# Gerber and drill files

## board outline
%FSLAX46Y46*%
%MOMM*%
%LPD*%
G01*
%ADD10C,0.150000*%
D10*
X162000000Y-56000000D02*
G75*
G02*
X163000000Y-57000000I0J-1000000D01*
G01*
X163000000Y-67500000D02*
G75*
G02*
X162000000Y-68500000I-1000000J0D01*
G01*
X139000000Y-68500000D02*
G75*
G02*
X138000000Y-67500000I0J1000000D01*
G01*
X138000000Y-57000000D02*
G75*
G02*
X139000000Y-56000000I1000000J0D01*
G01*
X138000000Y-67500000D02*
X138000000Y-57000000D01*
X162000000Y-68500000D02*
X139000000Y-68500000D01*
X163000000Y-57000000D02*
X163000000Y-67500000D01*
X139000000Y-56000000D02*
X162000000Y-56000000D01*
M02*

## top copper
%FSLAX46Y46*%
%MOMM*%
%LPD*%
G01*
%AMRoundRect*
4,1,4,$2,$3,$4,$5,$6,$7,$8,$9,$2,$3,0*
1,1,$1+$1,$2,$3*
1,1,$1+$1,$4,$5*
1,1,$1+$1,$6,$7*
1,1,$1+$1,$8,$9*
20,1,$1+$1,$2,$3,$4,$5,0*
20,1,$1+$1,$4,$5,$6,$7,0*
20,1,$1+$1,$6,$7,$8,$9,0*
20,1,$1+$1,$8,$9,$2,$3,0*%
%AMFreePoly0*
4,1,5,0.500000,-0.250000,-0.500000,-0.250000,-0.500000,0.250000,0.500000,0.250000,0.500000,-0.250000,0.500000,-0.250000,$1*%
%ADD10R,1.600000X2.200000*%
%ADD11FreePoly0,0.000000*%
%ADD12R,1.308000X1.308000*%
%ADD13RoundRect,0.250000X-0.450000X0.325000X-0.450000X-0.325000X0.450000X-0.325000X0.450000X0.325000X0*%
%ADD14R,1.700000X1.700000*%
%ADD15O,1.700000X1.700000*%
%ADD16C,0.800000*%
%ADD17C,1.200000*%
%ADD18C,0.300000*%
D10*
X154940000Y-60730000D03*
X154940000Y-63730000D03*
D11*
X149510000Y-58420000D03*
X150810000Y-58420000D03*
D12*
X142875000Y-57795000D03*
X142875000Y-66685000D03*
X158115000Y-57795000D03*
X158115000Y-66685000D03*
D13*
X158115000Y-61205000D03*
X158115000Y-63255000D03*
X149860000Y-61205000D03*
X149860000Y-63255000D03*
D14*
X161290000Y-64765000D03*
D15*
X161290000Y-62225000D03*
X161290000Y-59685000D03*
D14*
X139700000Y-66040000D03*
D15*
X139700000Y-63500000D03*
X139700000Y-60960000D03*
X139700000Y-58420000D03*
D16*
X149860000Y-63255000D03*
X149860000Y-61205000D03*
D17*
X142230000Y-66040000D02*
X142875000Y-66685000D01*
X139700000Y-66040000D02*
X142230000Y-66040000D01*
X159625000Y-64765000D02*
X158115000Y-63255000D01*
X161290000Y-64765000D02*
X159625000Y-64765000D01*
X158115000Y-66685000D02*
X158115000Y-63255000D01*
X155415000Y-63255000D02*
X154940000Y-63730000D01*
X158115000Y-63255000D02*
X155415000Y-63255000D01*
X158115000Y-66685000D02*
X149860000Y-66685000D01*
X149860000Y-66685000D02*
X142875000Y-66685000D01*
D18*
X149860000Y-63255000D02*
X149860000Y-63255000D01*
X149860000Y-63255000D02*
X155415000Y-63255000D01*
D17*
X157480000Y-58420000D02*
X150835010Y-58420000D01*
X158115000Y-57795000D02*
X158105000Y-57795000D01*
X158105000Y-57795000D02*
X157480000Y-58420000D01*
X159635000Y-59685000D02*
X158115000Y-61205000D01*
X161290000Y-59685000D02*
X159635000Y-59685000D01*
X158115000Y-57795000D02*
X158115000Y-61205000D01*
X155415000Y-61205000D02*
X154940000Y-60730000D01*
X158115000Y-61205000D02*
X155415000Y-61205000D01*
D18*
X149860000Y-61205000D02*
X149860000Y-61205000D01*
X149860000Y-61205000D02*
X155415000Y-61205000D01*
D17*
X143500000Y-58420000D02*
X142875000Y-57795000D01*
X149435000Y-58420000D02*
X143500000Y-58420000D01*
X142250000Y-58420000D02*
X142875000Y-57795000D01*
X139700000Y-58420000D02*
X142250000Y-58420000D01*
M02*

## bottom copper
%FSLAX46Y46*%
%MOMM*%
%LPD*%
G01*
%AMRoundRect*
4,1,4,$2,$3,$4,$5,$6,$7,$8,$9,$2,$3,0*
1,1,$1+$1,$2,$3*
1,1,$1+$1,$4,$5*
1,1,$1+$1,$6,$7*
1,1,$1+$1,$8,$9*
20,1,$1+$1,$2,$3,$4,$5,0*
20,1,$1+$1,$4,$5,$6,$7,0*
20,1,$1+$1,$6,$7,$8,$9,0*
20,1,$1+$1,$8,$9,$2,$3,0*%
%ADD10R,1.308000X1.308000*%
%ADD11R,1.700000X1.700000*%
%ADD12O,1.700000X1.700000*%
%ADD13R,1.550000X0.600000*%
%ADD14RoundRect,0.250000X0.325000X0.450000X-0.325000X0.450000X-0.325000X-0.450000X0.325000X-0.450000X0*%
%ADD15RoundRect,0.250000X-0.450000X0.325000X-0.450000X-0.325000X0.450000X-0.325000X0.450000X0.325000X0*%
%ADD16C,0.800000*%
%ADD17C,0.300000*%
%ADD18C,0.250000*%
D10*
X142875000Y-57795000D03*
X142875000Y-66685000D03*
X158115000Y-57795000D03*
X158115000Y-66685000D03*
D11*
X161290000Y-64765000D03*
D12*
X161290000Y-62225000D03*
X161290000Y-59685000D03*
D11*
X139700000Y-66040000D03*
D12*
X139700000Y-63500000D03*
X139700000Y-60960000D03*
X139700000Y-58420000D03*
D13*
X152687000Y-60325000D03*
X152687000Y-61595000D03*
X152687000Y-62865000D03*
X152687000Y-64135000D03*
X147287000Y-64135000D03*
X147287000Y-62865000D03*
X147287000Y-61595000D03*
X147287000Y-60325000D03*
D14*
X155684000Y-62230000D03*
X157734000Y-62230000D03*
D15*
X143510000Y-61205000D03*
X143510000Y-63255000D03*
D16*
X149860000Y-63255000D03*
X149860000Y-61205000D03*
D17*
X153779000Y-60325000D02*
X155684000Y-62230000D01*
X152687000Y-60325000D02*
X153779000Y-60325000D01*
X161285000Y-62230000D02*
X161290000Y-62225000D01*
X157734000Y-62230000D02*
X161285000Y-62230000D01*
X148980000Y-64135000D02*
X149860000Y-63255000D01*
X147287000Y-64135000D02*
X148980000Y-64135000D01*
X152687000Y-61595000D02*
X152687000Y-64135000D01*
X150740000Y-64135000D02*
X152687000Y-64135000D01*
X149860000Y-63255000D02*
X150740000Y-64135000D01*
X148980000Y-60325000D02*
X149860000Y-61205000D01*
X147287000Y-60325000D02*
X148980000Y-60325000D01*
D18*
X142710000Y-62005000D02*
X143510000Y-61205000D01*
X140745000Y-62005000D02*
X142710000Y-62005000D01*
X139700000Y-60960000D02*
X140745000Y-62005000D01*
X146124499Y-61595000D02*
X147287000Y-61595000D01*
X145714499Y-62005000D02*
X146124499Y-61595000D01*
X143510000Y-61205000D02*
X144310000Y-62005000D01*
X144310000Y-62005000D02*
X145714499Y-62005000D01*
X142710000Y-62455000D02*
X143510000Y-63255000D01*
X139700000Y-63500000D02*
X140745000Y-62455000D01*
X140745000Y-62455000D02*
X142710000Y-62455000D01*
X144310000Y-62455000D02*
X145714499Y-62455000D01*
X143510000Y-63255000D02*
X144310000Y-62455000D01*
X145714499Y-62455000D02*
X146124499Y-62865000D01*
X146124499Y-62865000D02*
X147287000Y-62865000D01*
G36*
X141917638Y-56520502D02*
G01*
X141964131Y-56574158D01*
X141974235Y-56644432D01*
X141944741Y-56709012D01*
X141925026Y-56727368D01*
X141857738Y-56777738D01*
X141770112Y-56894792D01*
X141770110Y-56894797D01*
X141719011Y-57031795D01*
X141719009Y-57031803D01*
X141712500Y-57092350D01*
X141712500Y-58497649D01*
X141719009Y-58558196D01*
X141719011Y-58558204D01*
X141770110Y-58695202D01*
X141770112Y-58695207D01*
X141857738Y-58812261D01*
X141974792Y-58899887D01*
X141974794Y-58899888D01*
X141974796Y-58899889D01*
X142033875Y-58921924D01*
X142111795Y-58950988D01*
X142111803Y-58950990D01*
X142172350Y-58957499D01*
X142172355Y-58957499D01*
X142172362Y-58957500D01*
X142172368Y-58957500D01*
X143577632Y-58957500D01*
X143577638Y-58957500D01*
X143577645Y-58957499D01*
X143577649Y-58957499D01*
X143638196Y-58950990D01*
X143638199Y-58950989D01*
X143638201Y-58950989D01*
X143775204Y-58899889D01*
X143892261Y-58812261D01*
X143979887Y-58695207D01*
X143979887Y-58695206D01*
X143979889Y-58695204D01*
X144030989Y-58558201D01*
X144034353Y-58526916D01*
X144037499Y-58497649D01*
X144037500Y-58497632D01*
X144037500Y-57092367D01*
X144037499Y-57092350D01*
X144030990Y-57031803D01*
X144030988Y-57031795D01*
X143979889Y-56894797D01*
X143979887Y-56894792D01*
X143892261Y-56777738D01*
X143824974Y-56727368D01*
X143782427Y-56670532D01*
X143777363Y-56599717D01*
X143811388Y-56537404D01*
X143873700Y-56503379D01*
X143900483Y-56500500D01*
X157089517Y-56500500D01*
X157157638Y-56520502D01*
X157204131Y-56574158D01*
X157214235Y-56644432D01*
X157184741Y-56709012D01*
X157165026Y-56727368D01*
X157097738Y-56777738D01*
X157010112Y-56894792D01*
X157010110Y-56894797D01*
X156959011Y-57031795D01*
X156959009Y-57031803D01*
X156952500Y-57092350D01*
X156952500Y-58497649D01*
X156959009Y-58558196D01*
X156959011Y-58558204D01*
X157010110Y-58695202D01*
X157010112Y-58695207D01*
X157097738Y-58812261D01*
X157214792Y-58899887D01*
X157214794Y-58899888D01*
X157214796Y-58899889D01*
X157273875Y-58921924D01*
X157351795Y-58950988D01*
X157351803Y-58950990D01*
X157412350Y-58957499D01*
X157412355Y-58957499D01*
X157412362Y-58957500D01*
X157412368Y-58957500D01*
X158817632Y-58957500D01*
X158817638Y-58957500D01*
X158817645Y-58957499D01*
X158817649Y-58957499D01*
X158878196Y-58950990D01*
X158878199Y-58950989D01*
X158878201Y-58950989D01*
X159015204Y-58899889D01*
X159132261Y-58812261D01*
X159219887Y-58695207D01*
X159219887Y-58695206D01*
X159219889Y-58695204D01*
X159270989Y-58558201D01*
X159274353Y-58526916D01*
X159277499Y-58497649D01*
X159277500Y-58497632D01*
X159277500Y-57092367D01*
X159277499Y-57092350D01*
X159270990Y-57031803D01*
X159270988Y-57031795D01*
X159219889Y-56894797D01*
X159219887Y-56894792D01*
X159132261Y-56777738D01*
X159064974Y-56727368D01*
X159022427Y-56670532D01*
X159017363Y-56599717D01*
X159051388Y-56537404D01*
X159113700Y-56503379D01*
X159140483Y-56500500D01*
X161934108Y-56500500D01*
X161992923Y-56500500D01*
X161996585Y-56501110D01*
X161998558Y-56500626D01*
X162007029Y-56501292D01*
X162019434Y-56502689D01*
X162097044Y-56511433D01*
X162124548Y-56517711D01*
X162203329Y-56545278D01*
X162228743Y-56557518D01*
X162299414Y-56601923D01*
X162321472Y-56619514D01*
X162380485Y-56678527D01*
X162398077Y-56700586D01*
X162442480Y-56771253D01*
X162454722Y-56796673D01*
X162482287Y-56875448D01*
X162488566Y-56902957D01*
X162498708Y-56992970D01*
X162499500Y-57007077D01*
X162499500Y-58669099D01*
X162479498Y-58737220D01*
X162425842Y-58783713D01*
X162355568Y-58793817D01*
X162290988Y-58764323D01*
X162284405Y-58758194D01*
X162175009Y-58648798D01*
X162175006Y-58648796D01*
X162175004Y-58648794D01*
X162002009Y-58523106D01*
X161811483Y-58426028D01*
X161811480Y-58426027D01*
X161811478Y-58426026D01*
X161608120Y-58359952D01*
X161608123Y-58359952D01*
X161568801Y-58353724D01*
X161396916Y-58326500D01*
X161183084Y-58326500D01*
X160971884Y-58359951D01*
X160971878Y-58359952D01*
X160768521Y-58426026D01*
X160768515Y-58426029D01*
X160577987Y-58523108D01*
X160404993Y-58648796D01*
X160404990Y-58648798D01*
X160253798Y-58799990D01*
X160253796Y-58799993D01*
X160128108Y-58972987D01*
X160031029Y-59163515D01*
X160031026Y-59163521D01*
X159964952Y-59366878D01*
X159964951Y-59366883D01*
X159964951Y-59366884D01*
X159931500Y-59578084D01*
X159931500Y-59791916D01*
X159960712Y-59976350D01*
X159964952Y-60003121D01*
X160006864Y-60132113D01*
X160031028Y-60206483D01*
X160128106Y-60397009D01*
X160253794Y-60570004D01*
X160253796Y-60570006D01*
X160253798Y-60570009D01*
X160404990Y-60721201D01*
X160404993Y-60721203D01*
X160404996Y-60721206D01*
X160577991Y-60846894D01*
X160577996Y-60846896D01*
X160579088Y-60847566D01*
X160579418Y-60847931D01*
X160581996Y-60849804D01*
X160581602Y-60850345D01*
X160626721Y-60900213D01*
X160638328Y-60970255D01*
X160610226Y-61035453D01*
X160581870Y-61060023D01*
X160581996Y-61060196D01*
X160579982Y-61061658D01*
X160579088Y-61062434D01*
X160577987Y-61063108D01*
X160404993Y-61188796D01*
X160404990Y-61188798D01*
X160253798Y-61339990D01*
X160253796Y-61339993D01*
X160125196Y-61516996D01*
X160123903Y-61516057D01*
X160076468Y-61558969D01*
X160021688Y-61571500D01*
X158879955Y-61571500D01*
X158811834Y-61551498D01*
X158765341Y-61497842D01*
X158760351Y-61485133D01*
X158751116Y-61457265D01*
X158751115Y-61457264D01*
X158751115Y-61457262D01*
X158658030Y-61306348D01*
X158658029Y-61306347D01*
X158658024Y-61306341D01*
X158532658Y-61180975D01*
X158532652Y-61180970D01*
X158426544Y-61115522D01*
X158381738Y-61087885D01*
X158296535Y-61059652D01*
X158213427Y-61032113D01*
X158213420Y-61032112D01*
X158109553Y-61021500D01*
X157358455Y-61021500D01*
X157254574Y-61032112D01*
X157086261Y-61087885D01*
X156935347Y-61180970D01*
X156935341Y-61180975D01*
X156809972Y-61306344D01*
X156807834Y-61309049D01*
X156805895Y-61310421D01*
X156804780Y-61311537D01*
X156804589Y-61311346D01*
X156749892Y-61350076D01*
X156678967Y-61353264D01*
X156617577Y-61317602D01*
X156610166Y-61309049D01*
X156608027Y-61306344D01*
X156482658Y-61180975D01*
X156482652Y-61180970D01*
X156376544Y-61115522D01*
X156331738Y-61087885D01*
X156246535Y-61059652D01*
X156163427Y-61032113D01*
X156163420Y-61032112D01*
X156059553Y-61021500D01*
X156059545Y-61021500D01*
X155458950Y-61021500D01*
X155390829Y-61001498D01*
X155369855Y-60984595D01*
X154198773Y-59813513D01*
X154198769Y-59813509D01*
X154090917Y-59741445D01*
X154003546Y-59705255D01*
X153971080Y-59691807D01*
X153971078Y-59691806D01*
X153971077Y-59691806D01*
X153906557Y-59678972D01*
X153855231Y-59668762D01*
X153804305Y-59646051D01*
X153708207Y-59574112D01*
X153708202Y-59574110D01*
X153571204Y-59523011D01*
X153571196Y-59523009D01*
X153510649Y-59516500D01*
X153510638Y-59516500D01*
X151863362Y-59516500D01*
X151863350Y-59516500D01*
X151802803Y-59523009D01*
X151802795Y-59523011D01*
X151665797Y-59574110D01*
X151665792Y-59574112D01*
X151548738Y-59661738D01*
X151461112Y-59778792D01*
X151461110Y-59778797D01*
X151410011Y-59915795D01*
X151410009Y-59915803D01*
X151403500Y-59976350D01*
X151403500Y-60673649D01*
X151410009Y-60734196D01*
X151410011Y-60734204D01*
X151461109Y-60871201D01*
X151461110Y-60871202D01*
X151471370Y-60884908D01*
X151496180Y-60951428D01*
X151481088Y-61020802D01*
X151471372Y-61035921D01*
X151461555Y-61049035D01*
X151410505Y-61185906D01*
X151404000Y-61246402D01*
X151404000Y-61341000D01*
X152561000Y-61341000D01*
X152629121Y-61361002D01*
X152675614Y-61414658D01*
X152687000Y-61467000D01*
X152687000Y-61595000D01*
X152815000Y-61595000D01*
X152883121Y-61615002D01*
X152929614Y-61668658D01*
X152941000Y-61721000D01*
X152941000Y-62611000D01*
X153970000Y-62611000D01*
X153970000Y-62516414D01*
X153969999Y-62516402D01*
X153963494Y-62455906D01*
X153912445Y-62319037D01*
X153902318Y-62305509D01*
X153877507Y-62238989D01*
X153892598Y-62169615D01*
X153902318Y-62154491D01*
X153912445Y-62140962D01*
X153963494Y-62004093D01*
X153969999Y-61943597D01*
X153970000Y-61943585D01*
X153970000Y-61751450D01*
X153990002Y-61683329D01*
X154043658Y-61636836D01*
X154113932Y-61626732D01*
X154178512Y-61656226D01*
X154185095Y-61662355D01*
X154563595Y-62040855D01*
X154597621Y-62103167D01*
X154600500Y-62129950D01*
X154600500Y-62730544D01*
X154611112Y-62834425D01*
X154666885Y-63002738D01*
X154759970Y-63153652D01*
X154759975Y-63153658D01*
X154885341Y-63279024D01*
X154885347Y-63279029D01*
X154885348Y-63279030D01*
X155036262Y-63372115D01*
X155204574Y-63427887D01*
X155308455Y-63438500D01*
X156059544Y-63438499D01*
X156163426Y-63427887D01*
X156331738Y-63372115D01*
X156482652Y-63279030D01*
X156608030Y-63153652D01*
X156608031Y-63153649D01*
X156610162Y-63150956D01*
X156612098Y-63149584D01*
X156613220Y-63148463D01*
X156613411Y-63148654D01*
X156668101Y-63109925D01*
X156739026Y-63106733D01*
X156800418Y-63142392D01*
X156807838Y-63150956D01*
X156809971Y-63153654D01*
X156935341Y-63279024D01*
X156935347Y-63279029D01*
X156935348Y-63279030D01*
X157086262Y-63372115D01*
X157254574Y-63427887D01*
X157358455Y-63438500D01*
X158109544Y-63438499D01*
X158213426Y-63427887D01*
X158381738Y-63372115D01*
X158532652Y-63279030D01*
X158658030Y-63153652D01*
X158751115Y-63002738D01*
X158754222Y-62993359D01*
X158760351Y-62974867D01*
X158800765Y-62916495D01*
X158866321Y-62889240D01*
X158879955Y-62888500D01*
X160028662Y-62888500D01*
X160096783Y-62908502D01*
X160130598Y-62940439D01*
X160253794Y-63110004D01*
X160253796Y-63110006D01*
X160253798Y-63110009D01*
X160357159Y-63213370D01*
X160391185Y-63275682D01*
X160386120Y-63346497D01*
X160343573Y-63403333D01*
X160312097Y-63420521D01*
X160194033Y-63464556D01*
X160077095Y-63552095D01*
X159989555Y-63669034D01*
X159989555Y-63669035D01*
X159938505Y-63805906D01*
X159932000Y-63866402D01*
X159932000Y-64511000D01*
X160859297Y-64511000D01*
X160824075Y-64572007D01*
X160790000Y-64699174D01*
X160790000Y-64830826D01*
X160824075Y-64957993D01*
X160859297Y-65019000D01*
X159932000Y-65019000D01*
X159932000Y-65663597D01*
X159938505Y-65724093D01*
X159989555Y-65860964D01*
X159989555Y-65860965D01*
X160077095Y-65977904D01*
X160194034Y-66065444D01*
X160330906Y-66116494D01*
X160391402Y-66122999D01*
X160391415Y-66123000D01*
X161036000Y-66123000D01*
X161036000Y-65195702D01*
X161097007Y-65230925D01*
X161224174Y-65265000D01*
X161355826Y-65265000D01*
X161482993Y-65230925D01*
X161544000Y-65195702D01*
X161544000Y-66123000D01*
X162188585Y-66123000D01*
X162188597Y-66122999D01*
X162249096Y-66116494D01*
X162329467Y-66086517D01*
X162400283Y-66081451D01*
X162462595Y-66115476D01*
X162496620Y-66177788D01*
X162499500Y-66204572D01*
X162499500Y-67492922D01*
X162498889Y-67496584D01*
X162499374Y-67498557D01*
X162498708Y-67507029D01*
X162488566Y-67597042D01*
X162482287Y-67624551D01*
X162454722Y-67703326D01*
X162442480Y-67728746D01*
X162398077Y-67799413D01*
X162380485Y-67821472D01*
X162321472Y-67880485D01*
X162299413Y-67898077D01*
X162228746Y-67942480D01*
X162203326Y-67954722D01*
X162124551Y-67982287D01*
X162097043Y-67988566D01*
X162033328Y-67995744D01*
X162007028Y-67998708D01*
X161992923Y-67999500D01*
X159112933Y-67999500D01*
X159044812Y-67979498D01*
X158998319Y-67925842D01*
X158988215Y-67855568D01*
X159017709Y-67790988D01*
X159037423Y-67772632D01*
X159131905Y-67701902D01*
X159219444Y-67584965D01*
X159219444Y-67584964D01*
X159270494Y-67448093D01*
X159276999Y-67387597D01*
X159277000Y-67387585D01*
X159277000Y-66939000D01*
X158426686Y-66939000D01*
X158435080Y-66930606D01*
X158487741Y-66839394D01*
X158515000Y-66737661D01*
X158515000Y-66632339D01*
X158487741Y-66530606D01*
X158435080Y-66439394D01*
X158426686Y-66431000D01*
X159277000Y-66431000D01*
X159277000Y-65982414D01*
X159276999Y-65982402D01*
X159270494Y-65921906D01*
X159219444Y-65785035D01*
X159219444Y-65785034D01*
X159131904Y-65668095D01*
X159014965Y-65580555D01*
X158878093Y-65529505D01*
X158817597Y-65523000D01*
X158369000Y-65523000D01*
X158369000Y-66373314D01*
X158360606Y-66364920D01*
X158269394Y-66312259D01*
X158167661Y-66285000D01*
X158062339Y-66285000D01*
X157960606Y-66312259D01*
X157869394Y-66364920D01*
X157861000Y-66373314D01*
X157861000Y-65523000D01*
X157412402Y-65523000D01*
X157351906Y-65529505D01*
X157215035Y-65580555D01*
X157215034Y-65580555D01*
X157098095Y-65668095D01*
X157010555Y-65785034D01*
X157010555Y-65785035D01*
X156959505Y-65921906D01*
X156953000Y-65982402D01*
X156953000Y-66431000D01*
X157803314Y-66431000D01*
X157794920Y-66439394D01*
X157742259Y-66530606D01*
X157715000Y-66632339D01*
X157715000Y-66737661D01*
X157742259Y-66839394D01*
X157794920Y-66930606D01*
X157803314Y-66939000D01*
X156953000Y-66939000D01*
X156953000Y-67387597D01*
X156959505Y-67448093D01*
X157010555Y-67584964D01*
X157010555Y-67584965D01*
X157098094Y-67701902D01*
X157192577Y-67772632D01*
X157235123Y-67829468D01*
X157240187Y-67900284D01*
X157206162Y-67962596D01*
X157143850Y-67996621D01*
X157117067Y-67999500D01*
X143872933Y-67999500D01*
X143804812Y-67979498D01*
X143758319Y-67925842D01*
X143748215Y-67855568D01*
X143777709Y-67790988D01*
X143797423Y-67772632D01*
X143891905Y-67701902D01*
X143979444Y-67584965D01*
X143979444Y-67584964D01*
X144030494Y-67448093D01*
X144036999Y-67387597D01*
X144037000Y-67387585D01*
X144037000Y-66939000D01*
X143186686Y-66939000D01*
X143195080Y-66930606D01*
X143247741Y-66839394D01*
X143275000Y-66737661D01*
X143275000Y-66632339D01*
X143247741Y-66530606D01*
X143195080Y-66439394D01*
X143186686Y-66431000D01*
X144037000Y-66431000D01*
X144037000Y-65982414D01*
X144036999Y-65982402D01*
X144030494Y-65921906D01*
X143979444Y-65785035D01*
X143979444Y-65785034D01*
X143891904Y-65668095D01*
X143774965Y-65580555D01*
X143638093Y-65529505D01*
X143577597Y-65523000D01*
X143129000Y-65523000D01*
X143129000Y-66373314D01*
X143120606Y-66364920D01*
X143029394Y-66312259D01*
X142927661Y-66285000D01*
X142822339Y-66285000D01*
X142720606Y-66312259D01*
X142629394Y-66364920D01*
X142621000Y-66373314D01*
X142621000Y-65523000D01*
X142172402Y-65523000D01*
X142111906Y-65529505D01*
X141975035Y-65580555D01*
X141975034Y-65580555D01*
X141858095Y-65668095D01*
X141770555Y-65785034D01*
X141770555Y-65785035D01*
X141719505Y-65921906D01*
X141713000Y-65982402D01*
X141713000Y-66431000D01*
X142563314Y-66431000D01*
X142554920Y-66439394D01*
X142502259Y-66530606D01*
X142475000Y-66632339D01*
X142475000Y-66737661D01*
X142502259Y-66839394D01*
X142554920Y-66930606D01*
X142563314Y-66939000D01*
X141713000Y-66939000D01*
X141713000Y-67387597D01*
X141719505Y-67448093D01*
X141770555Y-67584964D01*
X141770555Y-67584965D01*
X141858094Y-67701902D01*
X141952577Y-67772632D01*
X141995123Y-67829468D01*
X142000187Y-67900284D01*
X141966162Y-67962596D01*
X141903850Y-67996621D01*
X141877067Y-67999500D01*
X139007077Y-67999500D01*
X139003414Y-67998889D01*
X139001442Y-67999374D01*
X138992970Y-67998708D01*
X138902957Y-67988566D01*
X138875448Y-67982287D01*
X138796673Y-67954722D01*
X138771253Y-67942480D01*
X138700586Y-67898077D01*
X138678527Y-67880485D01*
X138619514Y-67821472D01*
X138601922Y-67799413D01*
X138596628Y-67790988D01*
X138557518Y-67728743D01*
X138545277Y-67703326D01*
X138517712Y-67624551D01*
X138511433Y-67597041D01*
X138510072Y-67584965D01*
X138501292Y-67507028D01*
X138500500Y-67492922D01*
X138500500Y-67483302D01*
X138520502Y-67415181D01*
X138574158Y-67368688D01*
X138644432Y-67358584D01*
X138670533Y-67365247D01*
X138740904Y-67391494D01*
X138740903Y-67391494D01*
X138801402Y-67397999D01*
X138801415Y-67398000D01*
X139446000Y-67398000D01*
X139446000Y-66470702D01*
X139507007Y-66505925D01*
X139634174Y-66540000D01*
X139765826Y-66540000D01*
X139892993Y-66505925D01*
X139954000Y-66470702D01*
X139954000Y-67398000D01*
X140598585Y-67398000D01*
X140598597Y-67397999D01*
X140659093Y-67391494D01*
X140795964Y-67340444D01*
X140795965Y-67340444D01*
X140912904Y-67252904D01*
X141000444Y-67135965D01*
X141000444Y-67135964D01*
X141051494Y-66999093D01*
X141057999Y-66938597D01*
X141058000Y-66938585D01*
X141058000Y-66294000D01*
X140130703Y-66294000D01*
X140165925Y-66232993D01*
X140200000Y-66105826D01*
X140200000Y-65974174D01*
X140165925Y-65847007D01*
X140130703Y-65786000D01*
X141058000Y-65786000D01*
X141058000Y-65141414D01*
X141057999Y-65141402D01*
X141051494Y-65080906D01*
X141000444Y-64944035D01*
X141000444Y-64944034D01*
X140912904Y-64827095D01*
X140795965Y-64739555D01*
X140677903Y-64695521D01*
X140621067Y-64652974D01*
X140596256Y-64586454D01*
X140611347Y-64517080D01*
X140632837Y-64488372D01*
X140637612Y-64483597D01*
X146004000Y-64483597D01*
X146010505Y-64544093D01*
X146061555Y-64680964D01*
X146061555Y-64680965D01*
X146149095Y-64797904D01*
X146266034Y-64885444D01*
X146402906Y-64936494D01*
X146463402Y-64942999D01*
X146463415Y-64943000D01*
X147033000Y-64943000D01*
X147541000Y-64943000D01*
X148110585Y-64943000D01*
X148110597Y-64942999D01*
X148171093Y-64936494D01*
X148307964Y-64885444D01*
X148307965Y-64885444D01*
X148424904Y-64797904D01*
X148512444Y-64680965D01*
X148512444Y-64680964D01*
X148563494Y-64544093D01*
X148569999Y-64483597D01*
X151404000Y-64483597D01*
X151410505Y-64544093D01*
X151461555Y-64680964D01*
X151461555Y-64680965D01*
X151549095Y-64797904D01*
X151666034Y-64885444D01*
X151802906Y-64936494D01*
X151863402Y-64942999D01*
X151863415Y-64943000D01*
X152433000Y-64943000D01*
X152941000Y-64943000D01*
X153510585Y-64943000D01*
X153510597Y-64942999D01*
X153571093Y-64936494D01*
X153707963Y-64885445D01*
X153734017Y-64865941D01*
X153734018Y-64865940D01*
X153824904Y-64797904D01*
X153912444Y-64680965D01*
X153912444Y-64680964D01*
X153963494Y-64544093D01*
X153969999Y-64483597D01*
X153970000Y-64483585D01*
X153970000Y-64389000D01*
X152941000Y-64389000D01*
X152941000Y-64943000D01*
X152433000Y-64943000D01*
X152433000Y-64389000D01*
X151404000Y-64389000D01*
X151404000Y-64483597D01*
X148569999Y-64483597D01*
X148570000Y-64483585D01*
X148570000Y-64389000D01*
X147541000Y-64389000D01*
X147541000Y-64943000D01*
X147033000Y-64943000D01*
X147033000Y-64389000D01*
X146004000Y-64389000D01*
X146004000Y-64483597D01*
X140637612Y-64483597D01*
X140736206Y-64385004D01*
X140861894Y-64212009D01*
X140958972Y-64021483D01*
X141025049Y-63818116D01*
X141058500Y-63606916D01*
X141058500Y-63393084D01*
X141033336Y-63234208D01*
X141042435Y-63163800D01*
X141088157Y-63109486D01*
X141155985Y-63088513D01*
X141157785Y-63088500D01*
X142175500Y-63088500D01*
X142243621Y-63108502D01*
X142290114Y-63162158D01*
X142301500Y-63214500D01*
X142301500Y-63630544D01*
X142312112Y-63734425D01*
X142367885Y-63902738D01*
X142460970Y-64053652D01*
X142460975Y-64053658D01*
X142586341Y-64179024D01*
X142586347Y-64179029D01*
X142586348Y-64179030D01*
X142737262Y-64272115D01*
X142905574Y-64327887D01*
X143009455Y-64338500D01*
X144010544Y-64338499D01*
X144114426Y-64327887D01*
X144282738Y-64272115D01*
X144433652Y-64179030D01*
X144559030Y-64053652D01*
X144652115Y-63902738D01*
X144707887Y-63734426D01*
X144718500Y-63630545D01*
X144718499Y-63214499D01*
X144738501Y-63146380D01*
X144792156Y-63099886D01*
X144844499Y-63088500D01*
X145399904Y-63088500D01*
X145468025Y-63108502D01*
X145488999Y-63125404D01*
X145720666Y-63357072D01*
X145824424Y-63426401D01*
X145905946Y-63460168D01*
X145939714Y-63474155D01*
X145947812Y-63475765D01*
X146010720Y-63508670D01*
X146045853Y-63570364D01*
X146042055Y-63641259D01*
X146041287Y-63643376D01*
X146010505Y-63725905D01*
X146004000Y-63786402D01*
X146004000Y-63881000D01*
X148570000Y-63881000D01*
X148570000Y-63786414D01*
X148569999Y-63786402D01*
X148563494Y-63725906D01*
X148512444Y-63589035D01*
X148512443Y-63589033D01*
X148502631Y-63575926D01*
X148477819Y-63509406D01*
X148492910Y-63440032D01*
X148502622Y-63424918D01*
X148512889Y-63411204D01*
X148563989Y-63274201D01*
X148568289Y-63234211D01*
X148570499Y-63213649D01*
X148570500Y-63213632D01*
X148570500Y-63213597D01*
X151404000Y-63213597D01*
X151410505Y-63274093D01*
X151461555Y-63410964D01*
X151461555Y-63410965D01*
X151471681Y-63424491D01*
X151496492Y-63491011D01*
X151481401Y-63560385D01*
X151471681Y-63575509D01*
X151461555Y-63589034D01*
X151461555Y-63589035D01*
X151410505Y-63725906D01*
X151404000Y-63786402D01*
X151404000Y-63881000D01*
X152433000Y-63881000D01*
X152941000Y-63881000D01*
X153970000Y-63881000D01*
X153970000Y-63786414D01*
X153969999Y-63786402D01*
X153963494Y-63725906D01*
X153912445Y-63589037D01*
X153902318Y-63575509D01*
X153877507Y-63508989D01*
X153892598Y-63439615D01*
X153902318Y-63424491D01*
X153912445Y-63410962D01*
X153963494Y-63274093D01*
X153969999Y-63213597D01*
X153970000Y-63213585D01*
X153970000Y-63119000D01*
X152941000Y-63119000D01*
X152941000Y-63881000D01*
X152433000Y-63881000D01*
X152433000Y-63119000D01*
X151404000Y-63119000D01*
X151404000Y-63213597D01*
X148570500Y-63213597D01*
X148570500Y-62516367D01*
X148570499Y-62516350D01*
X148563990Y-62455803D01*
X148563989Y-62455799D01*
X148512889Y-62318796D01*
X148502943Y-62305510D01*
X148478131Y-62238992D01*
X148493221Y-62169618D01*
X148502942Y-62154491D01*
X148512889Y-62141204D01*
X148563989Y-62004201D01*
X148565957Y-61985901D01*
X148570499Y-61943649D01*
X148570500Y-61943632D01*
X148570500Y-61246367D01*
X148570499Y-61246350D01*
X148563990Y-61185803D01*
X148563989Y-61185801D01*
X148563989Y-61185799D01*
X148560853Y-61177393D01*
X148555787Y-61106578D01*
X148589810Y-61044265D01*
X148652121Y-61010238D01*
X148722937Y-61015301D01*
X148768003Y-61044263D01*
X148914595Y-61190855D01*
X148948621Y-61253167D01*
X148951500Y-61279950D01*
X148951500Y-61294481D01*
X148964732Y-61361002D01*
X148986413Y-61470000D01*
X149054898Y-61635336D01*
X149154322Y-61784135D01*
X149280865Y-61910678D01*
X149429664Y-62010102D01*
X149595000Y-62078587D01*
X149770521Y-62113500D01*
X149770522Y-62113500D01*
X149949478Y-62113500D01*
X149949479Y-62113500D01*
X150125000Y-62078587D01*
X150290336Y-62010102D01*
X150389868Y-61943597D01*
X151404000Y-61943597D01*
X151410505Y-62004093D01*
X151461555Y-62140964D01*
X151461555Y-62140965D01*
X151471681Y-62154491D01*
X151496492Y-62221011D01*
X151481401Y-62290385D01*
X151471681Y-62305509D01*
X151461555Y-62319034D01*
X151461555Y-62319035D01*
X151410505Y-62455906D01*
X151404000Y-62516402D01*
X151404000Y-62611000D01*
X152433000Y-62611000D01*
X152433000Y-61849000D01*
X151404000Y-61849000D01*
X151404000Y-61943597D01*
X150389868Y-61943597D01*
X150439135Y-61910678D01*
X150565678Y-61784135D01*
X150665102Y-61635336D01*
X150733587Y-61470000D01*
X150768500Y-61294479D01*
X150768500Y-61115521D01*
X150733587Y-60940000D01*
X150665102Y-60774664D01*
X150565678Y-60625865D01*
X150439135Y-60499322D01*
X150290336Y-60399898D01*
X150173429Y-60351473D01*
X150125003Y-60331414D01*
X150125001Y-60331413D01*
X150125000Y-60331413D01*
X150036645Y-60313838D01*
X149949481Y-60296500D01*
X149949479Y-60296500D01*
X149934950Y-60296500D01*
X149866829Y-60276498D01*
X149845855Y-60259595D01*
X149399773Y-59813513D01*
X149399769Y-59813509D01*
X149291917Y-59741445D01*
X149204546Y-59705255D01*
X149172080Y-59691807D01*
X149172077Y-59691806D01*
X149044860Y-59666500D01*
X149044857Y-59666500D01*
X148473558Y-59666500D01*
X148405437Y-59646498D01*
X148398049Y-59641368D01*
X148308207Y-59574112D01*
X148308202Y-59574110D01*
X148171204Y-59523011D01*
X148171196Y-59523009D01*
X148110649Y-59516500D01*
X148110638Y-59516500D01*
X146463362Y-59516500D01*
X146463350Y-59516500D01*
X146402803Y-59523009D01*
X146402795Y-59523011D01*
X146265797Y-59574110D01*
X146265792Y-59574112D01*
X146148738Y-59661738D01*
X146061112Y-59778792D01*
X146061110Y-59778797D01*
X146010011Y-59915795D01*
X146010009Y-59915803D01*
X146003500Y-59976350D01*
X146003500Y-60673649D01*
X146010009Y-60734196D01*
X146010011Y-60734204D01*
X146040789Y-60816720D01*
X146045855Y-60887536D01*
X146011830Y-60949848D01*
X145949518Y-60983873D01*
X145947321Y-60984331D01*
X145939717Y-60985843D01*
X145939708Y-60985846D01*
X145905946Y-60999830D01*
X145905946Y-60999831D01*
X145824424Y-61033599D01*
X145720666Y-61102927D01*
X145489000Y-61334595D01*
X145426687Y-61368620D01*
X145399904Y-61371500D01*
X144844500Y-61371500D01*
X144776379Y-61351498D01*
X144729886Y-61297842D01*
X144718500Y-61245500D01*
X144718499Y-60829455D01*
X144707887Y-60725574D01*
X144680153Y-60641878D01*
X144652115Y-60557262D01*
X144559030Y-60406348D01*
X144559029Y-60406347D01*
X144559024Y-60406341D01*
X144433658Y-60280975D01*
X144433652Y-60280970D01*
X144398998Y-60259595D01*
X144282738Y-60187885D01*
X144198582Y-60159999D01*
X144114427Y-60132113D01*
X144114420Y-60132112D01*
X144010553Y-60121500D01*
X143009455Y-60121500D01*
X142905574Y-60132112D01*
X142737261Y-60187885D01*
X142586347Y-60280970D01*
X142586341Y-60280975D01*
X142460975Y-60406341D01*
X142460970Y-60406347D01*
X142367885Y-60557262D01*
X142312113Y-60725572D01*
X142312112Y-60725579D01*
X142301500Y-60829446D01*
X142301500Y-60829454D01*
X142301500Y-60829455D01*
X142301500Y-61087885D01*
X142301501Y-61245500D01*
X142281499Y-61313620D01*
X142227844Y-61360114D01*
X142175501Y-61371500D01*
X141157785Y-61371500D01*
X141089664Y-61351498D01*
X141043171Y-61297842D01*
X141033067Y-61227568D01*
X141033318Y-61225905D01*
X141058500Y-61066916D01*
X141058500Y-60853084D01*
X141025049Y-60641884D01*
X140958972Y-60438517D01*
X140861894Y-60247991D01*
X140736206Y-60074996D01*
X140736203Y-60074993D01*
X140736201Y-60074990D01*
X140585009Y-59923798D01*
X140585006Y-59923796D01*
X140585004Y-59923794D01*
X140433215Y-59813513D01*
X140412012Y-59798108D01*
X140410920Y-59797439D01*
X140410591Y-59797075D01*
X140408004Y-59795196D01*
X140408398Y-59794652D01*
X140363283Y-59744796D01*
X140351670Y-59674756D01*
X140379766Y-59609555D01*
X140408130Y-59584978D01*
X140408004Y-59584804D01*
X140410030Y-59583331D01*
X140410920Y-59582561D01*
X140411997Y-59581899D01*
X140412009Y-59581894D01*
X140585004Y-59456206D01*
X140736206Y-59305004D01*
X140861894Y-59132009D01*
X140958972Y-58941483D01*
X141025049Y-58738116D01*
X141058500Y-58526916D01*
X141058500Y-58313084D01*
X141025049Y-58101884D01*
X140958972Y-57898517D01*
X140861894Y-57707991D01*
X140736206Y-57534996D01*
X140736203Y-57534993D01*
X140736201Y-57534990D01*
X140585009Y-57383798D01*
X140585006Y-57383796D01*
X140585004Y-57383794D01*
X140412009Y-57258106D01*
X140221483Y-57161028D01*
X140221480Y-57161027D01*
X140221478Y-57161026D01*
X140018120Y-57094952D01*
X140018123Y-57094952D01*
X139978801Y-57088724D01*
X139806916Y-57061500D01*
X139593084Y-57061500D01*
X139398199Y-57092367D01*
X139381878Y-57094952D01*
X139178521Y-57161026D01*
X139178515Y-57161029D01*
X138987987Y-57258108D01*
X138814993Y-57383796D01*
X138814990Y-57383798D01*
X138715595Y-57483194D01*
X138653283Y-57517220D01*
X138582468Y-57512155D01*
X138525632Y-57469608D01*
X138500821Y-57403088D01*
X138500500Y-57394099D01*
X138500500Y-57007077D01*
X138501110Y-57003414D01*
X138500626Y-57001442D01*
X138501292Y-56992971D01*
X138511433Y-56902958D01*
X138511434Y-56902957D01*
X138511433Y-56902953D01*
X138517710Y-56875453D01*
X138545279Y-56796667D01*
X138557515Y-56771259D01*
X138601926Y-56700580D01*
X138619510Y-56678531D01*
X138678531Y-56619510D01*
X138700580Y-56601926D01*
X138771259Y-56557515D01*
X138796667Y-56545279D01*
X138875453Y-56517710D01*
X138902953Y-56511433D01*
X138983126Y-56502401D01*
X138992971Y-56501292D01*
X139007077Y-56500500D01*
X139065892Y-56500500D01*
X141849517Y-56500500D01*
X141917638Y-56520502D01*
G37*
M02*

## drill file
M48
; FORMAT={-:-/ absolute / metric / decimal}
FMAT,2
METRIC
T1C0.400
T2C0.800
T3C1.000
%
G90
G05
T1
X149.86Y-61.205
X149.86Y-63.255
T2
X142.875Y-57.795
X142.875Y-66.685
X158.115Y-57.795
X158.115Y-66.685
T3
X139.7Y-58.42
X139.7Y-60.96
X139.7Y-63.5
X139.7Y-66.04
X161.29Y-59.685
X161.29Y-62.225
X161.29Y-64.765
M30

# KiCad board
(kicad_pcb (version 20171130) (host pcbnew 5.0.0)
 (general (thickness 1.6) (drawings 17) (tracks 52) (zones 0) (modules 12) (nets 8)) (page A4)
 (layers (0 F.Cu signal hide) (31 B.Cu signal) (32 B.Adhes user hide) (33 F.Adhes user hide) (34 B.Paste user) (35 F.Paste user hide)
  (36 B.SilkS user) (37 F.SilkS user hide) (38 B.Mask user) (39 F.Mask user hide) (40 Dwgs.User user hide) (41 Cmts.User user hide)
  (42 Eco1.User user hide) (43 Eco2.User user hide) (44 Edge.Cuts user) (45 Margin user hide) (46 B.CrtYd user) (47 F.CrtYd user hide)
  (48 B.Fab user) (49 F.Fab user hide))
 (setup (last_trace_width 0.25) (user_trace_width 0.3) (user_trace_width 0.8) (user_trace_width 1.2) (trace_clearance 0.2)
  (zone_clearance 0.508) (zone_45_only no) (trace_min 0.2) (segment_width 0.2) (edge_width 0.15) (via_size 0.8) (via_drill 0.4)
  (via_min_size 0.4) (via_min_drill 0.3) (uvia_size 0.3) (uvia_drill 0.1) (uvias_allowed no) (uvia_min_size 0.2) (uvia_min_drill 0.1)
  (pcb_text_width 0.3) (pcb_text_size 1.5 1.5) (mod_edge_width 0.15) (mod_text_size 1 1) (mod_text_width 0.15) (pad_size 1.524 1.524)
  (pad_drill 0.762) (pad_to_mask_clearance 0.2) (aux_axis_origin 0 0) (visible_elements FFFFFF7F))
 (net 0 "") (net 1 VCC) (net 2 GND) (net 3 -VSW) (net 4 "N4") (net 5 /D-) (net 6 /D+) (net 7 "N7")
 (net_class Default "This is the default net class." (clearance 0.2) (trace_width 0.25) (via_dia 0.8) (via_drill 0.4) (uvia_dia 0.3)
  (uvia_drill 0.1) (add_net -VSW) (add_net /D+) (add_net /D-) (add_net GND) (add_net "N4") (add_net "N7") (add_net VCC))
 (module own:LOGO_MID (layer B.Cu) (at 159.004 65.532 180)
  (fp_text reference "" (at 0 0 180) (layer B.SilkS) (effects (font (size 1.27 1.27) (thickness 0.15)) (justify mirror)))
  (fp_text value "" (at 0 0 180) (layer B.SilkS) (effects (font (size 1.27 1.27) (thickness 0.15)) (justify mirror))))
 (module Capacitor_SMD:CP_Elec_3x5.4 (layer F.Cu) (at 154.94 62.23 270)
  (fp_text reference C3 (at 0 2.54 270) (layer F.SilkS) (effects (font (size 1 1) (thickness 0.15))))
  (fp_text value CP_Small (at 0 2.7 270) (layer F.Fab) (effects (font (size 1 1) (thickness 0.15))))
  (pad 1 smd rect (at -1.5 0 270) (size 2.2 1.6) (layers F.Cu F.Paste F.Mask) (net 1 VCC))
  (pad 2 smd rect (at 1.5 0 270) (size 2.2 1.6) (layers F.Cu F.Paste F.Mask) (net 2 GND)))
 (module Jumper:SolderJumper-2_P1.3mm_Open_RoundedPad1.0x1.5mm (layer F.Cu) (at 150.16 58.42)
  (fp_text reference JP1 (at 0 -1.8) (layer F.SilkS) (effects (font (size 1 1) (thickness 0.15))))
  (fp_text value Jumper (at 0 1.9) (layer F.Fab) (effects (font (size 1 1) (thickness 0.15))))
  (pad 1 smd custom (at -0.65 0) (size 1 0.5) (layers F.Cu F.Mask) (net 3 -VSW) (zone_connect 0) (options (clearance outline) (anchor rect))
   (primitives))
  (pad 2 smd custom (at 0.65 0) (size 1 0.5) (layers F.Cu F.Mask) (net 1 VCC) (zone_connect 0) (options (clearance outline) (anchor rect))
   (primitives)))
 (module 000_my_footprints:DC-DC (layer F.Cu) (at 142.875 57.795)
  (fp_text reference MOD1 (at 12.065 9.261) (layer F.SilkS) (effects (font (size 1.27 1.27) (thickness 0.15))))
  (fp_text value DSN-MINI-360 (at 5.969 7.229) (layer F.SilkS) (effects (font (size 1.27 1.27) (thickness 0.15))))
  (pad IN thru_hole rect (at 0 0) (size 1.308 1.308) (drill 0.8) (layers *.Cu *.Mask) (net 3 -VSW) (solder_mask_margin 0.1016))
  (pad GND thru_hole rect (at 0 8.89) (size 1.308 1.308) (drill 0.8) (layers *.Cu *.Mask) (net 2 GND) (solder_mask_margin 0.1016))
  (pad OUT thru_hole rect (at 15.24 0) (size 1.308 1.308) (drill 0.8) (layers *.Cu *.Mask) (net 1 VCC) (solder_mask_margin 0.1016))
  (pad GND thru_hole rect (at 15.24 8.89) (size 1.308 1.308) (drill 0.8) (layers *.Cu *.Mask) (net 2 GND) (solder_mask_margin 0.1016)))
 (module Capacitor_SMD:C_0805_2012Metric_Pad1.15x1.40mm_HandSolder (layer F.Cu) (at 158.115 62.23 270)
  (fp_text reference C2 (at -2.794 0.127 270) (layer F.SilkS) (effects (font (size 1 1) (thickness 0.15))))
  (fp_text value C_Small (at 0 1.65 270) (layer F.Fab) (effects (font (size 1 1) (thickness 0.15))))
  (pad 1 smd roundrect (at -1.025 0 270) (size 1.15 1.4) (layers F.Cu F.Paste F.Mask) (roundrect_rratio 0.217391) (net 1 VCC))
  (pad 2 smd roundrect (at 1.025 0 270) (size 1.15 1.4) (layers F.Cu F.Paste F.Mask) (roundrect_rratio 0.217391) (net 2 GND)))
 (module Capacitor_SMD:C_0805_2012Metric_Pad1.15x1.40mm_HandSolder (layer F.Cu) (at 149.86 62.23 270)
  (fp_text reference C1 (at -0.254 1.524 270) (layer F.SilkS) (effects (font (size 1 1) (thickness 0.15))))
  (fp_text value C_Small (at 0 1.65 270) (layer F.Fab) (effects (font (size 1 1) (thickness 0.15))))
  (pad 1 smd roundrect (at -1.025 0 270) (size 1.15 1.4) (layers F.Cu F.Paste F.Mask) (roundrect_rratio 0.217391) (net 1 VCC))
  (pad 2 smd roundrect (at 1.025 0 270) (size 1.15 1.4) (layers F.Cu F.Paste F.Mask) (roundrect_rratio 0.217391) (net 2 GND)))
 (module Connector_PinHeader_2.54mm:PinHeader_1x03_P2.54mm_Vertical (layer F.Cu) (at 161.29 64.765 180)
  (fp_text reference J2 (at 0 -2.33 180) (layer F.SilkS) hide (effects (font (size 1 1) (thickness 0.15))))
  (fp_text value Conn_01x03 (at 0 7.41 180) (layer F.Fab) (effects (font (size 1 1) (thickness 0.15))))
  (pad 1 thru_hole rect (at 0 0 180) (size 1.7 1.7) (drill 1) (layers *.Cu *.Mask) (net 2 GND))
  (pad 2 thru_hole oval (at 0 2.54 180) (size 1.7 1.7) (drill 1) (layers *.Cu *.Mask) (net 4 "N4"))
  (pad 3 thru_hole oval (at 0 5.08 180) (size 1.7 1.7) (drill 1) (layers *.Cu *.Mask) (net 1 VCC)))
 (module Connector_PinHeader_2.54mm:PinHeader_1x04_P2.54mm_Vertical (layer F.Cu) (at 139.7 66.04 180)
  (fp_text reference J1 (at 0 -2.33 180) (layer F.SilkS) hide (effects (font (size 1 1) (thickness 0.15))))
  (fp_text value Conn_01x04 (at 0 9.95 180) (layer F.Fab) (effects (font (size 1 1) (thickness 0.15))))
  (pad 1 thru_hole rect (at 0 0 180) (size 1.7 1.7) (drill 1) (layers *.Cu *.Mask) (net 2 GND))
  (pad 2 thru_hole oval (at 0 2.54 180) (size 1.7 1.7) (drill 1) (layers *.Cu *.Mask) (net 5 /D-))
  (pad 3 thru_hole oval (at 0 5.08 180) (size 1.7 1.7) (drill 1) (layers *.Cu *.Mask) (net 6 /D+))
  (pad 4 thru_hole oval (at 0 7.62 180) (size 1.7 1.7) (drill 1) (layers *.Cu *.Mask) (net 3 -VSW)))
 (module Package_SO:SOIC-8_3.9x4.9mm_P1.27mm (layer B.Cu) (at 149.987 62.23 180)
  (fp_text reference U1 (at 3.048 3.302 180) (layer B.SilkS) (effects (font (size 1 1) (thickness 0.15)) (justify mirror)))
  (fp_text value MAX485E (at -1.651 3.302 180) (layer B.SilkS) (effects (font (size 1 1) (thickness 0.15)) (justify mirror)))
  (pad 1 smd rect (at -2.7 1.905 180) (size 1.55 0.6) (layers B.Cu B.Paste B.Mask) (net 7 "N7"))
  (pad 2 smd rect (at -2.7 0.635 180) (size 1.55 0.6) (layers B.Cu B.Paste B.Mask) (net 2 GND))
  (pad 3 smd rect (at -2.7 -0.635 180) (size 1.55 0.6) (layers B.Cu B.Paste B.Mask) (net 2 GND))
  (pad 4 smd rect (at -2.7 -1.905 180) (size 1.55 0.6) (layers B.Cu B.Paste B.Mask) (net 2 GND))
  (pad 5 smd rect (at 2.7 -1.905 180) (size 1.55 0.6) (layers B.Cu B.Paste B.Mask) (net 2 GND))
  (pad 6 smd rect (at 2.7 -0.635 180) (size 1.55 0.6) (layers B.Cu B.Paste B.Mask) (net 5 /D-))
  (pad 7 smd rect (at 2.7 0.635 180) (size 1.55 0.6) (layers B.Cu B.Paste B.Mask) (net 6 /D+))
  (pad 8 smd rect (at 2.7 1.905 180) (size 1.55 0.6) (layers B.Cu B.Paste B.Mask) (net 1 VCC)))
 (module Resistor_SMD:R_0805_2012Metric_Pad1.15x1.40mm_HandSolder (layer B.Cu) (at 156.709 62.23 180)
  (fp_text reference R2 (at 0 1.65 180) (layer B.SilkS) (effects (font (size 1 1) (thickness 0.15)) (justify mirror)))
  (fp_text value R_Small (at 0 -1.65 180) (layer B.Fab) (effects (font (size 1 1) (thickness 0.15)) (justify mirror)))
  (pad 2 smd roundrect (at 1.025 0 180) (size 1.15 1.4) (layers B.Cu B.Paste B.Mask) (roundrect_rratio 0.217391) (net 7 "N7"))
  (pad 1 smd roundrect (at -1.025 0 180) (size 1.15 1.4) (layers B.Cu B.Paste B.Mask) (roundrect_rratio 0.217391) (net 4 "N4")))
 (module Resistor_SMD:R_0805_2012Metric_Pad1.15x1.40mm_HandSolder (layer B.Cu) (at 143.51 62.23 270)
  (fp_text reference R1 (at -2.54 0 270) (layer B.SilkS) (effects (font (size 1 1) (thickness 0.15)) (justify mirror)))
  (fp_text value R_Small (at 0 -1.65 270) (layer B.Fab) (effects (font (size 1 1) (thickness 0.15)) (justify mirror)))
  (pad 1 smd roundrect (at -1.025 0 270) (size 1.15 1.4) (layers B.Cu B.Paste B.Mask) (roundrect_rratio 0.217391) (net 6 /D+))
  (pad 2 smd roundrect (at 1.025 0 270) (size 1.15 1.4) (layers B.Cu B.Paste B.Mask) (roundrect_rratio 0.217391) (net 5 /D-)))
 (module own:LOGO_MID (layer F.Cu) (at 146.812 60.706 180)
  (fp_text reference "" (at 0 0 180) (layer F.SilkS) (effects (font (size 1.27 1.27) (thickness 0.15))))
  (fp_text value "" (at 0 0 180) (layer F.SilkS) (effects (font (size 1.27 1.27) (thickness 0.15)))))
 (gr_arc (start 162 57) (end 163 57) (angle -90) (layer Edge.Cuts) (width 0.15))
 (gr_arc (start 162 67.5) (end 162 68.5) (angle -90) (layer Edge.Cuts) (width 0.15))
 (gr_arc (start 139 67.5) (end 138 67.5) (angle -90) (layer Edge.Cuts) (width 0.15))
 (gr_arc (start 139 57) (end 139 56) (angle -90) (layer Edge.Cuts) (width 0.15))
 (gr_line (start 138 67.5) (end 138 57) (layer Edge.Cuts) (width 0.15))
 (gr_line (start 162 68.5) (end 139 68.5) (layer Edge.Cuts) (width 0.15))
 (gr_line (start 163 57) (end 163 67.5) (layer Edge.Cuts) (width 0.15))
 (gr_line (start 139 56) (end 162 56) (layer Edge.Cuts) (width 0.15))
 (segment (start 153.779 60.325) (end 155.684 62.23) (width 0.3) (layer B.Cu) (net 7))
 (segment (start 152.687 60.325) (end 153.779 60.325) (width 0.3) (layer B.Cu) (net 7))
 (segment (start 161.285 62.23) (end 161.29 62.225) (width 0.3) (layer B.Cu) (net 4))
 (segment (start 157.734 62.23) (end 161.285 62.23) (width 0.3) (layer B.Cu) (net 4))
 (segment (start 142.23 66.04) (end 142.875 66.685) (width 1.2) (layer F.Cu) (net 2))
 (segment (start 139.7 66.04) (end 142.23 66.04) (width 1.2) (layer F.Cu) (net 2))
 (segment (start 159.625 64.765) (end 158.115 63.255) (width 1.2) (layer F.Cu) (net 2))
 (segment (start 161.29 64.765) (end 159.625 64.765) (width 1.2) (layer F.Cu) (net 2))
 (segment (start 158.115 66.685) (end 158.115 63.255) (width 1.2) (layer F.Cu) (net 2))
 (segment (start 155.415 63.255) (end 154.94 63.73) (width 1.2) (layer F.Cu) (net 2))
 (segment (start 158.115 63.255) (end 155.415 63.255) (width 1.2) (layer F.Cu) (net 2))
 (segment (start 158.115 66.685) (end 149.86 66.685) (width 1.2) (layer F.Cu) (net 2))
 (segment (start 149.86 66.685) (end 142.875 66.685) (width 1.2) (layer F.Cu) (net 2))
 (segment (start 149.86 63.255) (end 149.86 63.255) (width 0.3) (layer F.Cu) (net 2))
 (segment (start 149.86 63.255) (end 155.415 63.255) (width 0.3) (layer F.Cu) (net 2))
 (via (at 149.86 63.255) (size 0.8) (drill 0.4) (layers F.Cu B.Cu) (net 2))
 (segment (start 148.98 64.135) (end 149.86 63.255) (width 0.3) (layer B.Cu) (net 2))
 (segment (start 147.287 64.135) (end 148.98 64.135) (width 0.3) (layer B.Cu) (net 2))
 (segment (start 152.687 61.595) (end 152.687 64.135) (width 0.3) (layer B.Cu) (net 2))
 (segment (start 150.74 64.135) (end 152.687 64.135) (width 0.3) (layer B.Cu) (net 2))
 (segment (start 149.86 63.255) (end 150.74 64.135) (width 0.3) (layer B.Cu) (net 2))
 (segment (start 157.48 58.42) (end 150.83501 58.42) (width 1.2) (layer F.Cu) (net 1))
 (segment (start 158.115 57.795) (end 158.105 57.795) (width 1.2) (layer F.Cu) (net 1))
 (segment (start 158.105 57.795) (end 157.48 58.42) (width 1.2) (layer F.Cu) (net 1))
 (segment (start 159.635 59.685) (end 158.115 61.205) (width 1.2) (layer F.Cu) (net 1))
 (segment (start 161.29 59.685) (end 159.635 59.685) (width 1.2) (layer F.Cu) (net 1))
 (segment (start 158.115 57.795) (end 158.115 61.205) (width 1.2) (layer F.Cu) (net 1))
 (segment (start 155.415 61.205) (end 154.94 60.73) (width 1.2) (layer F.Cu) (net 1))
 (segment (start 158.115 61.205) (end 155.415 61.205) (width 1.2) (layer F.Cu) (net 1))
 (segment (start 149.86 61.205) (end 149.86 61.205) (width 0.3) (layer F.Cu) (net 1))
 (segment (start 149.86 61.205) (end 155.415 61.205) (width 0.3) (layer F.Cu) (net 1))
 (via (at 149.86 61.205) (size 0.8) (drill 0.4) (layers F.Cu B.Cu) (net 1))
 (segment (start 148.98 60.325) (end 149.86 61.205) (width 0.3) (layer B.Cu) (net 1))
 (segment (start 147.287 60.325) (end 148.98 60.325) (width 0.3) (layer B.Cu) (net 1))
 (segment (start 143.5 58.42) (end 142.875 57.795) (width 1.2) (layer F.Cu) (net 3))
 (segment (start 149.435 58.42) (end 143.5 58.42) (width 1.2) (layer F.Cu) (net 3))
 (segment (start 142.25 58.42) (end 142.875 57.795) (width 1.2) (layer F.Cu) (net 3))
 (segment (start 139.7 58.42) (end 142.25 58.42) (width 1.2) (layer F.Cu) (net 3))
 (segment (start 142.71 62.005) (end 143.51 61.205) (width 0.25) (layer B.Cu) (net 6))
 (segment (start 140.745 62.005) (end 142.71 62.005) (width 0.25) (layer B.Cu) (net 6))
 (segment (start 139.7 60.96) (end 140.745 62.005) (width 0.25) (layer B.Cu) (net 6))
 (segment (start 146.124499 61.595) (end 147.287 61.595) (width 0.25) (layer B.Cu) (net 6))
 (segment (start 145.714499 62.005) (end 146.124499 61.595) (width 0.25) (layer B.Cu) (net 6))
 (segment (start 143.51 61.205) (end 144.31 62.005) (width 0.25) (layer B.Cu) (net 6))
 (segment (start 144.31 62.005) (end 145.714499 62.005) (width 0.25) (layer B.Cu) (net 6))
 (segment (start 142.71 62.455) (end 143.51 63.255) (width 0.25) (layer B.Cu) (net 5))
 (segment (start 139.7 63.5) (end 140.745 62.455) (width 0.25) (layer B.Cu) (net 5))
 (segment (start 140.745 62.455) (end 142.71 62.455) (width 0.25) (layer B.Cu) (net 5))
 (segment (start 144.31 62.455) (end 145.714499 62.455) (width 0.25) (layer B.Cu) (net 5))
 (segment (start 143.51 63.255) (end 144.31 62.455) (width 0.25) (layer B.Cu) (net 5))
 (segment (start 145.714499 62.455) (end 146.124499 62.865) (width 0.25) (layer B.Cu) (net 5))
 (segment (start 146.124499 62.865) (end 147.287 62.865) (width 0.25) (layer B.Cu) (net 5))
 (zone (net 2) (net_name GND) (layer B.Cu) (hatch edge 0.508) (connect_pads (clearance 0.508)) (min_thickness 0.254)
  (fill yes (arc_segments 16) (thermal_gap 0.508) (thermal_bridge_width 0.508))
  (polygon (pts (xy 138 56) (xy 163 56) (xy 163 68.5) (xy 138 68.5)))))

